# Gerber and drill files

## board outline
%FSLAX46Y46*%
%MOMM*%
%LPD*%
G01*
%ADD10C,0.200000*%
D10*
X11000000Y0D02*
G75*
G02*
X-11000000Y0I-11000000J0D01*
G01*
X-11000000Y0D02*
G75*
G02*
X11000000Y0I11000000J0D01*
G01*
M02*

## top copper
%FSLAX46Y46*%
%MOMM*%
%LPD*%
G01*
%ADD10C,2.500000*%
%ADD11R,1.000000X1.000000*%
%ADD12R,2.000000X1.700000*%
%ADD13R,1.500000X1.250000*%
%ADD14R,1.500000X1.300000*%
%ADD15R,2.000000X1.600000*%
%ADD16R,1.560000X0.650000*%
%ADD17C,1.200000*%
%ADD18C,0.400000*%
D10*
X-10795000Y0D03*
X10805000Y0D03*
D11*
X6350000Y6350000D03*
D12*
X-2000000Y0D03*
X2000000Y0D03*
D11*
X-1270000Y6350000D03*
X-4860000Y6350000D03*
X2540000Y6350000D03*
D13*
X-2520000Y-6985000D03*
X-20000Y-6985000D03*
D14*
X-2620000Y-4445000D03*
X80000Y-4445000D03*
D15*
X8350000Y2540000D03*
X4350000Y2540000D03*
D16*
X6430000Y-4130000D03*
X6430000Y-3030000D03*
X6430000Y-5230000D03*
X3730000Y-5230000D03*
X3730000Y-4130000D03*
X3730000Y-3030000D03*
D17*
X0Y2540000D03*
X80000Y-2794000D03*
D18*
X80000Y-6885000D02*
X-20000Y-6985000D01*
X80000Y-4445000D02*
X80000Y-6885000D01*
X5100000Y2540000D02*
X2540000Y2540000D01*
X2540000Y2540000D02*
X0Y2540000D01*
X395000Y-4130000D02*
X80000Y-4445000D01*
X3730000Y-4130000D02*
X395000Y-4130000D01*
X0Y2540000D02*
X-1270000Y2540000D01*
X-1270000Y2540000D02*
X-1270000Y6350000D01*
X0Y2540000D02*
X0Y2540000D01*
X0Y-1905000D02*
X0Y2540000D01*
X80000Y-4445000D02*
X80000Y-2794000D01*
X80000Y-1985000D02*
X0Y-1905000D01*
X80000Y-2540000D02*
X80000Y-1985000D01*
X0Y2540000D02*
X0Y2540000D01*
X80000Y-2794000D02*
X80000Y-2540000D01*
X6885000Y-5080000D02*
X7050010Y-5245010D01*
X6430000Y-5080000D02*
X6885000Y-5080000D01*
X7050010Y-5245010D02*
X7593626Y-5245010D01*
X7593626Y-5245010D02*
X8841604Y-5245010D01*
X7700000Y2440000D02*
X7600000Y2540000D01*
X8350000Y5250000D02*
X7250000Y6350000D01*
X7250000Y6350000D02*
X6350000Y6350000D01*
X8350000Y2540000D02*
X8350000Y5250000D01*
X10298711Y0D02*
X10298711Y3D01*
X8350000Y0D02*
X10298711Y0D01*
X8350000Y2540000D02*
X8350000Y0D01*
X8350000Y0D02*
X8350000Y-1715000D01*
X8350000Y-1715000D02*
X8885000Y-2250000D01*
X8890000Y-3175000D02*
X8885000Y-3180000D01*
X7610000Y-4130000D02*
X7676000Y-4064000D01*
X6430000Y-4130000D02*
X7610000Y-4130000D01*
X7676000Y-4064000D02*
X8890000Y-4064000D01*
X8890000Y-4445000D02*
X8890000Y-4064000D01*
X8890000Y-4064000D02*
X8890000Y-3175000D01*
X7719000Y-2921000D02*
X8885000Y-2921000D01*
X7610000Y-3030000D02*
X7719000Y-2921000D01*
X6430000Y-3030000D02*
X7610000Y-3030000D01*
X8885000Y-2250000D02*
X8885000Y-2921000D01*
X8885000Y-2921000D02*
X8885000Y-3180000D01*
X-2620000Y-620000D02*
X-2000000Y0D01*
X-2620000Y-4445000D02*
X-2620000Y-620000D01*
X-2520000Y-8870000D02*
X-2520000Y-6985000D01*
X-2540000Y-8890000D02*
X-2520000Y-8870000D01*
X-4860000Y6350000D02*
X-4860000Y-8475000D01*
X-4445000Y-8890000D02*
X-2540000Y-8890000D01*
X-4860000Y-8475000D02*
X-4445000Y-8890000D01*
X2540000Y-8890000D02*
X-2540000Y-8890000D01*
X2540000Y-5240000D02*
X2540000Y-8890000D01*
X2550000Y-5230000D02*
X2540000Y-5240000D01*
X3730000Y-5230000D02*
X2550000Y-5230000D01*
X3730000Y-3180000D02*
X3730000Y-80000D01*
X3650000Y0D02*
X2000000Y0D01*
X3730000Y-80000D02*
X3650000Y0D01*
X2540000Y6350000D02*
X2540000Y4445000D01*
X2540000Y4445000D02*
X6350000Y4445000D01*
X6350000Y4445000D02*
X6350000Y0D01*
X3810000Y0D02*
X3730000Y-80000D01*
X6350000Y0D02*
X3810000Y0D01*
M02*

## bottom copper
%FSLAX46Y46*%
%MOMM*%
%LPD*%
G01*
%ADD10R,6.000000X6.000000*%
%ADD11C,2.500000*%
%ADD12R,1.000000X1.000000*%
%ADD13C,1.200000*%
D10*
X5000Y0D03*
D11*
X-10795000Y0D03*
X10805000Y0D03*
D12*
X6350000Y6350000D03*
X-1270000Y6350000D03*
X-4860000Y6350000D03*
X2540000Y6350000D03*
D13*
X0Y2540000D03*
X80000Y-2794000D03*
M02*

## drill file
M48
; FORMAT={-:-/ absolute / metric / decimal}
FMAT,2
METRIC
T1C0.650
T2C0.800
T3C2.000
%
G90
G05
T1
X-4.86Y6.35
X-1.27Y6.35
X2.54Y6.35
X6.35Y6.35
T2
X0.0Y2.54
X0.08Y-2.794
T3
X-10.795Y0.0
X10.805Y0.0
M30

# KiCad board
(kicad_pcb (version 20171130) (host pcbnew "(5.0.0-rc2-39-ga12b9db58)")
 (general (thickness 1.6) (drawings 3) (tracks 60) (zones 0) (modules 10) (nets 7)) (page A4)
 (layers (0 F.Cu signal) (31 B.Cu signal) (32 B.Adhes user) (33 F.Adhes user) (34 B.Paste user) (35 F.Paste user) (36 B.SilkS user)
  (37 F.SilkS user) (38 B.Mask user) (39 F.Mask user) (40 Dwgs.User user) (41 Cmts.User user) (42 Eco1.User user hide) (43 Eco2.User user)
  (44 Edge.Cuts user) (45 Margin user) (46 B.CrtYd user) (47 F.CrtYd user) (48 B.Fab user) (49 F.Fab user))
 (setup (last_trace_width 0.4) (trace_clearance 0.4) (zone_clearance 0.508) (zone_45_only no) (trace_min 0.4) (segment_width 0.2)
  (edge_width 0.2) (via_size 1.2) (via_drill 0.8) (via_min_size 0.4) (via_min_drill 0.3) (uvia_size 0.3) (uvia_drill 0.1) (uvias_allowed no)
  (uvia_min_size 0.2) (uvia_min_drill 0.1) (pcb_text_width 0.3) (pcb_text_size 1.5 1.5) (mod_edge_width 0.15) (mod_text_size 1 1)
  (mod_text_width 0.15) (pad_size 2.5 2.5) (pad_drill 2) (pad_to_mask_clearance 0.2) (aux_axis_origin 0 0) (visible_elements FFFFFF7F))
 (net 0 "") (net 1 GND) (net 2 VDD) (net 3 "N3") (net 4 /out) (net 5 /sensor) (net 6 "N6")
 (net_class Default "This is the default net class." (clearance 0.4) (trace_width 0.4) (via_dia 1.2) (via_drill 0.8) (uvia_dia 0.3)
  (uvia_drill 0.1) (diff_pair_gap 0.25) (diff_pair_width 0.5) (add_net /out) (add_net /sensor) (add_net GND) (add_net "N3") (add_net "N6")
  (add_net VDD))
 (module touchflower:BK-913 (layer B.Cu) (at 0.005 0)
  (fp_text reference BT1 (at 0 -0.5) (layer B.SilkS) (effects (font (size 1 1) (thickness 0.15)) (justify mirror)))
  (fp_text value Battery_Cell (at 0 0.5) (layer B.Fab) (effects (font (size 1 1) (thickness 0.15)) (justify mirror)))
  (pad 2 smd rect (at 0 0) (size 6 6) (layers B.Cu B.Paste B.Mask) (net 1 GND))
  (pad 1 thru_hole circle (at -10.8 0) (size 2.5 2.5) (drill 2) (layers *.Cu *.Mask) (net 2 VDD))
  (pad 1 thru_hole circle (at 10.8 0) (size 2.5 2.5) (drill 2) (layers *.Cu *.Mask) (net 2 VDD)))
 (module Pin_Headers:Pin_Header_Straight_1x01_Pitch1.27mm (layer F.Cu) (at 6.35 -6.35)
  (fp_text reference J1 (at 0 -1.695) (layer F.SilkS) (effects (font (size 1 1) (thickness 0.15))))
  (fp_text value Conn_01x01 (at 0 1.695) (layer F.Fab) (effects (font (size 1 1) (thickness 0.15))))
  (pad 1 thru_hole rect (at 0 0) (size 1 1) (drill 0.65) (layers *.Cu *.Mask) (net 2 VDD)))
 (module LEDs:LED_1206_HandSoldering (layer F.Cu) (at 0 0)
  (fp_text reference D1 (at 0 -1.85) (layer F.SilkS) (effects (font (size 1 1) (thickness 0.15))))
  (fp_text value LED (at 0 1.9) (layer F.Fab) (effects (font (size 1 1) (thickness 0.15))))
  (pad 1 smd rect (at -2 0) (size 2 1.7) (layers F.Cu F.Paste F.Mask) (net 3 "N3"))
  (pad 2 smd rect (at 2 0) (size 2 1.7) (layers F.Cu F.Paste F.Mask) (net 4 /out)))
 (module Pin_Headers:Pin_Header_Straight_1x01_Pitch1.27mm (layer F.Cu) (at -1.27 -6.35)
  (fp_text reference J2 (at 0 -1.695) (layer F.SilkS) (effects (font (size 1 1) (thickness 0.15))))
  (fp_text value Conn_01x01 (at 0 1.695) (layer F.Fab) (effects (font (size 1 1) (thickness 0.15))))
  (pad 1 thru_hole rect (at 0 0) (size 1 1) (drill 0.65) (layers *.Cu *.Mask) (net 1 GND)))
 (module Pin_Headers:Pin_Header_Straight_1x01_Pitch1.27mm (layer F.Cu) (at -4.86 -6.35)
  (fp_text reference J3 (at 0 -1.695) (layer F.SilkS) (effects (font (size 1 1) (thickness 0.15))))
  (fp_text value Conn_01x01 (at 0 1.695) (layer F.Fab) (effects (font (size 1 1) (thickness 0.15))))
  (pad 1 thru_hole rect (at 0 0) (size 1 1) (drill 0.65) (layers *.Cu *.Mask) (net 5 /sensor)))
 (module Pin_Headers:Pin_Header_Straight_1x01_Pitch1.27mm (layer F.Cu) (at 2.54 -6.35)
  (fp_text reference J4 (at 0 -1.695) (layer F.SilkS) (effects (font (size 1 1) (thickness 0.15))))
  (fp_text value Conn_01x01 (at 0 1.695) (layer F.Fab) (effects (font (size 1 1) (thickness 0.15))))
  (pad 1 thru_hole rect (at 0 0) (size 1 1) (drill 0.65) (layers *.Cu *.Mask) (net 4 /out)))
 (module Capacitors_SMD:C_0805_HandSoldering (layer F.Cu) (at -1.27 6.985)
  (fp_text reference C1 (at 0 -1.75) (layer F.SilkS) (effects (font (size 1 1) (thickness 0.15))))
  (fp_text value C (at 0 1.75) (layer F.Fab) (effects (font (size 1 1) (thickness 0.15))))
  (pad 1 smd rect (at -1.25 0) (size 1.5 1.25) (layers F.Cu F.Paste F.Mask) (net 5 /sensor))
  (pad 2 smd rect (at 1.25 0) (size 1.5 1.25) (layers F.Cu F.Paste F.Mask) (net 1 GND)))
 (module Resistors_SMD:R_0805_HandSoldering (layer F.Cu) (at -1.27 4.445)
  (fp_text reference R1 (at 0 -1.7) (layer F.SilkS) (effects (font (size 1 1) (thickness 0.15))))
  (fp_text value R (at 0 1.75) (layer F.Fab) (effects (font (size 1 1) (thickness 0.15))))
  (pad 1 smd rect (at -1.35 0) (size 1.5 1.3) (layers F.Cu F.Paste F.Mask) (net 3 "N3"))
  (pad 2 smd rect (at 1.35 0) (size 1.5 1.3) (layers F.Cu F.Paste F.Mask) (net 1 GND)))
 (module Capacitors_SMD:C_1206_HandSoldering (layer F.Cu) (at 6.35 -2.54 180)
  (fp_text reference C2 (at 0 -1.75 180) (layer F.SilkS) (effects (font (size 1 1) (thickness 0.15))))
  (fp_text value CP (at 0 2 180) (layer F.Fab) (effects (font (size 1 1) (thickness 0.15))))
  (pad 1 smd rect (at -2 0 180) (size 2 1.6) (layers F.Cu F.Paste F.Mask) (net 2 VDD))
  (pad 2 smd rect (at 2 0 180) (size 2 1.6) (layers F.Cu F.Paste F.Mask) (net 1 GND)))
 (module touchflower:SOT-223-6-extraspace (layer F.Cu) (at 5.08 4.13)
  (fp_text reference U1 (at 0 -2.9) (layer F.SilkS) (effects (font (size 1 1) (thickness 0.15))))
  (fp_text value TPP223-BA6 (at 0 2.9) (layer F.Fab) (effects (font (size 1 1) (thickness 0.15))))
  (pad 5 smd rect (at 1.35 0) (size 1.56 0.65) (layers F.Cu F.Paste F.Mask) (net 2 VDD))
  (pad 6 smd rect (at 1.35 -1.1) (size 1.56 0.65) (layers F.Cu F.Paste F.Mask) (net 2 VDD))
  (pad 4 smd rect (at 1.35 1.1) (size 1.56 0.65) (layers F.Cu F.Paste F.Mask) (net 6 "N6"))
  (pad 3 smd rect (at -1.35 1.1) (size 1.56 0.65) (layers F.Cu F.Paste F.Mask) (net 5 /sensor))
  (pad 2 smd rect (at -1.35 0) (size 1.56 0.65) (layers F.Cu F.Paste F.Mask) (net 1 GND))
  (pad 1 smd rect (at -1.35 -1.1) (size 1.56 0.65) (layers F.Cu F.Paste F.Mask) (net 4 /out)))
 (gr_circle (center 0 0) (end 11 0) (layer Edge.Cuts) (width 0.2))
 (segment (start 0.08 6.885) (end -0.02 6.985) (width 0.4) (layer F.Cu) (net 1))
 (segment (start 0.08 4.445) (end 0.08 6.885) (width 0.4) (layer F.Cu) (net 1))
 (segment (start 5.1 -2.54) (end 2.54 -2.54) (width 0.4) (layer F.Cu) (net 1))
 (segment (start 2.54 -2.54) (end 0 -2.54) (width 0.4) (layer F.Cu) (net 1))
 (segment (start 0.395 4.13) (end 0.08 4.445) (width 0.4) (layer F.Cu) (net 1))
 (segment (start 3.73 4.13) (end 0.395 4.13) (width 0.4) (layer F.Cu) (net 1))
 (segment (start 0 -2.54) (end -1.27 -2.54) (width 0.4) (layer F.Cu) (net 1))
 (segment (start -1.27 -2.54) (end -1.27 -6.35) (width 0.4) (layer F.Cu) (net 1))
 (segment (start 0 -2.54) (end 0 -2.54) (width 0.4) (layer F.Cu) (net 1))
 (segment (start 0 1.905) (end 0 -2.54) (width 0.4) (layer F.Cu) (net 1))
 (segment (start 0.08 4.445) (end 0.08 2.794) (width 0.4) (layer F.Cu) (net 1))
 (segment (start 0.08 1.985) (end 0 1.905) (width 0.4) (layer F.Cu) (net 1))
 (segment (start 0.08 2.54) (end 0.08 1.985) (width 0.4) (layer F.Cu) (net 1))
 (segment (start 0 -2.54) (end 0 -2.54) (width 0.4) (layer F.Cu) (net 1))
 (via (at 0 -2.54) (size 1.2) (drill 0.8) (layers F.Cu B.Cu) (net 1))
 (segment (start 0.08 2.794) (end 0.08 2.54) (width 0.4) (layer F.Cu) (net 1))
 (via (at 0.08 2.794) (size 1.2) (drill 0.8) (layers F.Cu B.Cu) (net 1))
 (segment (start 6.885 5.08) (end 7.05001 5.24501) (width 0.4) (layer F.Cu) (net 6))
 (segment (start 6.43 5.08) (end 6.885 5.08) (width 0.4) (layer F.Cu) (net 6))
 (segment (start 7.05001 5.24501) (end 7.593626 5.24501) (width 0.4) (layer F.Cu) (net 6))
 (segment (start 7.593626 5.24501) (end 8.841604 5.24501) (width 0.4) (layer F.Cu) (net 6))
 (segment (start 7.7 -2.44) (end 7.6 -2.54) (width 0.4) (layer F.Cu) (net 2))
 (segment (start 8.35 -5.25) (end 7.25 -6.35) (width 0.4) (layer F.Cu) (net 2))
 (segment (start 7.25 -6.35) (end 6.35 -6.35) (width 0.4) (layer F.Cu) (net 2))
 (segment (start 8.35 -2.54) (end 8.35 -5.25) (width 0.4) (layer F.Cu) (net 2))
 (segment (start 10.298711 0) (end 10.298711 -0.000003) (width 0.4) (layer F.Cu) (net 2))
 (segment (start 8.35 0) (end 10.298711 0) (width 0.4) (layer F.Cu) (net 2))
 (segment (start 8.35 -2.54) (end 8.35 0) (width 0.4) (layer F.Cu) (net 2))
 (segment (start 8.35 0) (end 8.35 1.715) (width 0.4) (layer F.Cu) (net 2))
 (segment (start 8.35 1.715) (end 8.885 2.25) (width 0.4) (layer F.Cu) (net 2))
 (segment (start 8.89 3.175) (end 8.885 3.18) (width 0.4) (layer F.Cu) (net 2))
 (segment (start 7.61 4.13) (end 7.676 4.064) (width 0.4) (layer F.Cu) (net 2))
 (segment (start 6.43 4.13) (end 7.61 4.13) (width 0.4) (layer F.Cu) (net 2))
 (segment (start 7.676 4.064) (end 8.89 4.064) (width 0.4) (layer F.Cu) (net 2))
 (segment (start 8.89 4.445) (end 8.89 4.064) (width 0.4) (layer F.Cu) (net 2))
 (segment (start 8.89 4.064) (end 8.89 3.175) (width 0.4) (layer F.Cu) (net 2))
 (segment (start 7.719 2.921) (end 8.885 2.921) (width 0.4) (layer F.Cu) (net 2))
 (segment (start 7.61 3.03) (end 7.719 2.921) (width 0.4) (layer F.Cu) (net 2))
 (segment (start 6.43 3.03) (end 7.61 3.03) (width 0.4) (layer F.Cu) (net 2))
 (segment (start 8.885 2.25) (end 8.885 2.921) (width 0.4) (layer F.Cu) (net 2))
 (segment (start 8.885 2.921) (end 8.885 3.18) (width 0.4) (layer F.Cu) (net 2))
 (segment (start -2.62 0.62) (end -2 0) (width 0.4) (layer F.Cu) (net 3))
 (segment (start -2.62 4.445) (end -2.62 0.62) (width 0.4) (layer F.Cu) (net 3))
 (segment (start -2.52 8.87) (end -2.52 6.985) (width 0.4) (layer F.Cu) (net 5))
 (segment (start -2.54 8.89) (end -2.52 8.87) (width 0.4) (layer F.Cu) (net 5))
 (segment (start -4.86 -6.35) (end -4.86 8.475) (width 0.4) (layer F.Cu) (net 5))
 (segment (start -4.445 8.89) (end -2.54 8.89) (width 0.4) (layer F.Cu) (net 5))
 (segment (start -4.86 8.475) (end -4.445 8.89) (width 0.4) (layer F.Cu) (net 5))
 (segment (start 2.54 8.89) (end -2.54 8.89) (width 0.4) (layer F.Cu) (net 5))
 (segment (start 2.54 5.24) (end 2.54 8.89) (width 0.4) (layer F.Cu) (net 5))
 (segment (start 2.55 5.23) (end 2.54 5.24) (width 0.4) (layer F.Cu) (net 5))
 (segment (start 3.73 5.23) (end 2.55 5.23) (width 0.4) (layer F.Cu) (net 5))
 (segment (start 3.73 3.18) (end 3.73 0.08) (width 0.4) (layer F.Cu) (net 4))
 (segment (start 3.65 0) (end 2 0) (width 0.4) (layer F.Cu) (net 4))
 (segment (start 3.73 0.08) (end 3.65 0) (width 0.4) (layer F.Cu) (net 4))
 (segment (start 2.54 -6.35) (end 2.54 -4.445) (width 0.4) (layer F.Cu) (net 4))
 (segment (start 2.54 -4.445) (end 6.35 -4.445) (width 0.4) (layer F.Cu) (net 4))
 (segment (start 6.35 -4.445) (end 6.35 0) (width 0.4) (layer F.Cu) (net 4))
 (segment (start 3.81 0) (end 3.73 0.08) (width 0.4) (layer F.Cu) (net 4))
 (segment (start 6.35 0) (end 3.81 0) (width 0.4) (layer F.Cu) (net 4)))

